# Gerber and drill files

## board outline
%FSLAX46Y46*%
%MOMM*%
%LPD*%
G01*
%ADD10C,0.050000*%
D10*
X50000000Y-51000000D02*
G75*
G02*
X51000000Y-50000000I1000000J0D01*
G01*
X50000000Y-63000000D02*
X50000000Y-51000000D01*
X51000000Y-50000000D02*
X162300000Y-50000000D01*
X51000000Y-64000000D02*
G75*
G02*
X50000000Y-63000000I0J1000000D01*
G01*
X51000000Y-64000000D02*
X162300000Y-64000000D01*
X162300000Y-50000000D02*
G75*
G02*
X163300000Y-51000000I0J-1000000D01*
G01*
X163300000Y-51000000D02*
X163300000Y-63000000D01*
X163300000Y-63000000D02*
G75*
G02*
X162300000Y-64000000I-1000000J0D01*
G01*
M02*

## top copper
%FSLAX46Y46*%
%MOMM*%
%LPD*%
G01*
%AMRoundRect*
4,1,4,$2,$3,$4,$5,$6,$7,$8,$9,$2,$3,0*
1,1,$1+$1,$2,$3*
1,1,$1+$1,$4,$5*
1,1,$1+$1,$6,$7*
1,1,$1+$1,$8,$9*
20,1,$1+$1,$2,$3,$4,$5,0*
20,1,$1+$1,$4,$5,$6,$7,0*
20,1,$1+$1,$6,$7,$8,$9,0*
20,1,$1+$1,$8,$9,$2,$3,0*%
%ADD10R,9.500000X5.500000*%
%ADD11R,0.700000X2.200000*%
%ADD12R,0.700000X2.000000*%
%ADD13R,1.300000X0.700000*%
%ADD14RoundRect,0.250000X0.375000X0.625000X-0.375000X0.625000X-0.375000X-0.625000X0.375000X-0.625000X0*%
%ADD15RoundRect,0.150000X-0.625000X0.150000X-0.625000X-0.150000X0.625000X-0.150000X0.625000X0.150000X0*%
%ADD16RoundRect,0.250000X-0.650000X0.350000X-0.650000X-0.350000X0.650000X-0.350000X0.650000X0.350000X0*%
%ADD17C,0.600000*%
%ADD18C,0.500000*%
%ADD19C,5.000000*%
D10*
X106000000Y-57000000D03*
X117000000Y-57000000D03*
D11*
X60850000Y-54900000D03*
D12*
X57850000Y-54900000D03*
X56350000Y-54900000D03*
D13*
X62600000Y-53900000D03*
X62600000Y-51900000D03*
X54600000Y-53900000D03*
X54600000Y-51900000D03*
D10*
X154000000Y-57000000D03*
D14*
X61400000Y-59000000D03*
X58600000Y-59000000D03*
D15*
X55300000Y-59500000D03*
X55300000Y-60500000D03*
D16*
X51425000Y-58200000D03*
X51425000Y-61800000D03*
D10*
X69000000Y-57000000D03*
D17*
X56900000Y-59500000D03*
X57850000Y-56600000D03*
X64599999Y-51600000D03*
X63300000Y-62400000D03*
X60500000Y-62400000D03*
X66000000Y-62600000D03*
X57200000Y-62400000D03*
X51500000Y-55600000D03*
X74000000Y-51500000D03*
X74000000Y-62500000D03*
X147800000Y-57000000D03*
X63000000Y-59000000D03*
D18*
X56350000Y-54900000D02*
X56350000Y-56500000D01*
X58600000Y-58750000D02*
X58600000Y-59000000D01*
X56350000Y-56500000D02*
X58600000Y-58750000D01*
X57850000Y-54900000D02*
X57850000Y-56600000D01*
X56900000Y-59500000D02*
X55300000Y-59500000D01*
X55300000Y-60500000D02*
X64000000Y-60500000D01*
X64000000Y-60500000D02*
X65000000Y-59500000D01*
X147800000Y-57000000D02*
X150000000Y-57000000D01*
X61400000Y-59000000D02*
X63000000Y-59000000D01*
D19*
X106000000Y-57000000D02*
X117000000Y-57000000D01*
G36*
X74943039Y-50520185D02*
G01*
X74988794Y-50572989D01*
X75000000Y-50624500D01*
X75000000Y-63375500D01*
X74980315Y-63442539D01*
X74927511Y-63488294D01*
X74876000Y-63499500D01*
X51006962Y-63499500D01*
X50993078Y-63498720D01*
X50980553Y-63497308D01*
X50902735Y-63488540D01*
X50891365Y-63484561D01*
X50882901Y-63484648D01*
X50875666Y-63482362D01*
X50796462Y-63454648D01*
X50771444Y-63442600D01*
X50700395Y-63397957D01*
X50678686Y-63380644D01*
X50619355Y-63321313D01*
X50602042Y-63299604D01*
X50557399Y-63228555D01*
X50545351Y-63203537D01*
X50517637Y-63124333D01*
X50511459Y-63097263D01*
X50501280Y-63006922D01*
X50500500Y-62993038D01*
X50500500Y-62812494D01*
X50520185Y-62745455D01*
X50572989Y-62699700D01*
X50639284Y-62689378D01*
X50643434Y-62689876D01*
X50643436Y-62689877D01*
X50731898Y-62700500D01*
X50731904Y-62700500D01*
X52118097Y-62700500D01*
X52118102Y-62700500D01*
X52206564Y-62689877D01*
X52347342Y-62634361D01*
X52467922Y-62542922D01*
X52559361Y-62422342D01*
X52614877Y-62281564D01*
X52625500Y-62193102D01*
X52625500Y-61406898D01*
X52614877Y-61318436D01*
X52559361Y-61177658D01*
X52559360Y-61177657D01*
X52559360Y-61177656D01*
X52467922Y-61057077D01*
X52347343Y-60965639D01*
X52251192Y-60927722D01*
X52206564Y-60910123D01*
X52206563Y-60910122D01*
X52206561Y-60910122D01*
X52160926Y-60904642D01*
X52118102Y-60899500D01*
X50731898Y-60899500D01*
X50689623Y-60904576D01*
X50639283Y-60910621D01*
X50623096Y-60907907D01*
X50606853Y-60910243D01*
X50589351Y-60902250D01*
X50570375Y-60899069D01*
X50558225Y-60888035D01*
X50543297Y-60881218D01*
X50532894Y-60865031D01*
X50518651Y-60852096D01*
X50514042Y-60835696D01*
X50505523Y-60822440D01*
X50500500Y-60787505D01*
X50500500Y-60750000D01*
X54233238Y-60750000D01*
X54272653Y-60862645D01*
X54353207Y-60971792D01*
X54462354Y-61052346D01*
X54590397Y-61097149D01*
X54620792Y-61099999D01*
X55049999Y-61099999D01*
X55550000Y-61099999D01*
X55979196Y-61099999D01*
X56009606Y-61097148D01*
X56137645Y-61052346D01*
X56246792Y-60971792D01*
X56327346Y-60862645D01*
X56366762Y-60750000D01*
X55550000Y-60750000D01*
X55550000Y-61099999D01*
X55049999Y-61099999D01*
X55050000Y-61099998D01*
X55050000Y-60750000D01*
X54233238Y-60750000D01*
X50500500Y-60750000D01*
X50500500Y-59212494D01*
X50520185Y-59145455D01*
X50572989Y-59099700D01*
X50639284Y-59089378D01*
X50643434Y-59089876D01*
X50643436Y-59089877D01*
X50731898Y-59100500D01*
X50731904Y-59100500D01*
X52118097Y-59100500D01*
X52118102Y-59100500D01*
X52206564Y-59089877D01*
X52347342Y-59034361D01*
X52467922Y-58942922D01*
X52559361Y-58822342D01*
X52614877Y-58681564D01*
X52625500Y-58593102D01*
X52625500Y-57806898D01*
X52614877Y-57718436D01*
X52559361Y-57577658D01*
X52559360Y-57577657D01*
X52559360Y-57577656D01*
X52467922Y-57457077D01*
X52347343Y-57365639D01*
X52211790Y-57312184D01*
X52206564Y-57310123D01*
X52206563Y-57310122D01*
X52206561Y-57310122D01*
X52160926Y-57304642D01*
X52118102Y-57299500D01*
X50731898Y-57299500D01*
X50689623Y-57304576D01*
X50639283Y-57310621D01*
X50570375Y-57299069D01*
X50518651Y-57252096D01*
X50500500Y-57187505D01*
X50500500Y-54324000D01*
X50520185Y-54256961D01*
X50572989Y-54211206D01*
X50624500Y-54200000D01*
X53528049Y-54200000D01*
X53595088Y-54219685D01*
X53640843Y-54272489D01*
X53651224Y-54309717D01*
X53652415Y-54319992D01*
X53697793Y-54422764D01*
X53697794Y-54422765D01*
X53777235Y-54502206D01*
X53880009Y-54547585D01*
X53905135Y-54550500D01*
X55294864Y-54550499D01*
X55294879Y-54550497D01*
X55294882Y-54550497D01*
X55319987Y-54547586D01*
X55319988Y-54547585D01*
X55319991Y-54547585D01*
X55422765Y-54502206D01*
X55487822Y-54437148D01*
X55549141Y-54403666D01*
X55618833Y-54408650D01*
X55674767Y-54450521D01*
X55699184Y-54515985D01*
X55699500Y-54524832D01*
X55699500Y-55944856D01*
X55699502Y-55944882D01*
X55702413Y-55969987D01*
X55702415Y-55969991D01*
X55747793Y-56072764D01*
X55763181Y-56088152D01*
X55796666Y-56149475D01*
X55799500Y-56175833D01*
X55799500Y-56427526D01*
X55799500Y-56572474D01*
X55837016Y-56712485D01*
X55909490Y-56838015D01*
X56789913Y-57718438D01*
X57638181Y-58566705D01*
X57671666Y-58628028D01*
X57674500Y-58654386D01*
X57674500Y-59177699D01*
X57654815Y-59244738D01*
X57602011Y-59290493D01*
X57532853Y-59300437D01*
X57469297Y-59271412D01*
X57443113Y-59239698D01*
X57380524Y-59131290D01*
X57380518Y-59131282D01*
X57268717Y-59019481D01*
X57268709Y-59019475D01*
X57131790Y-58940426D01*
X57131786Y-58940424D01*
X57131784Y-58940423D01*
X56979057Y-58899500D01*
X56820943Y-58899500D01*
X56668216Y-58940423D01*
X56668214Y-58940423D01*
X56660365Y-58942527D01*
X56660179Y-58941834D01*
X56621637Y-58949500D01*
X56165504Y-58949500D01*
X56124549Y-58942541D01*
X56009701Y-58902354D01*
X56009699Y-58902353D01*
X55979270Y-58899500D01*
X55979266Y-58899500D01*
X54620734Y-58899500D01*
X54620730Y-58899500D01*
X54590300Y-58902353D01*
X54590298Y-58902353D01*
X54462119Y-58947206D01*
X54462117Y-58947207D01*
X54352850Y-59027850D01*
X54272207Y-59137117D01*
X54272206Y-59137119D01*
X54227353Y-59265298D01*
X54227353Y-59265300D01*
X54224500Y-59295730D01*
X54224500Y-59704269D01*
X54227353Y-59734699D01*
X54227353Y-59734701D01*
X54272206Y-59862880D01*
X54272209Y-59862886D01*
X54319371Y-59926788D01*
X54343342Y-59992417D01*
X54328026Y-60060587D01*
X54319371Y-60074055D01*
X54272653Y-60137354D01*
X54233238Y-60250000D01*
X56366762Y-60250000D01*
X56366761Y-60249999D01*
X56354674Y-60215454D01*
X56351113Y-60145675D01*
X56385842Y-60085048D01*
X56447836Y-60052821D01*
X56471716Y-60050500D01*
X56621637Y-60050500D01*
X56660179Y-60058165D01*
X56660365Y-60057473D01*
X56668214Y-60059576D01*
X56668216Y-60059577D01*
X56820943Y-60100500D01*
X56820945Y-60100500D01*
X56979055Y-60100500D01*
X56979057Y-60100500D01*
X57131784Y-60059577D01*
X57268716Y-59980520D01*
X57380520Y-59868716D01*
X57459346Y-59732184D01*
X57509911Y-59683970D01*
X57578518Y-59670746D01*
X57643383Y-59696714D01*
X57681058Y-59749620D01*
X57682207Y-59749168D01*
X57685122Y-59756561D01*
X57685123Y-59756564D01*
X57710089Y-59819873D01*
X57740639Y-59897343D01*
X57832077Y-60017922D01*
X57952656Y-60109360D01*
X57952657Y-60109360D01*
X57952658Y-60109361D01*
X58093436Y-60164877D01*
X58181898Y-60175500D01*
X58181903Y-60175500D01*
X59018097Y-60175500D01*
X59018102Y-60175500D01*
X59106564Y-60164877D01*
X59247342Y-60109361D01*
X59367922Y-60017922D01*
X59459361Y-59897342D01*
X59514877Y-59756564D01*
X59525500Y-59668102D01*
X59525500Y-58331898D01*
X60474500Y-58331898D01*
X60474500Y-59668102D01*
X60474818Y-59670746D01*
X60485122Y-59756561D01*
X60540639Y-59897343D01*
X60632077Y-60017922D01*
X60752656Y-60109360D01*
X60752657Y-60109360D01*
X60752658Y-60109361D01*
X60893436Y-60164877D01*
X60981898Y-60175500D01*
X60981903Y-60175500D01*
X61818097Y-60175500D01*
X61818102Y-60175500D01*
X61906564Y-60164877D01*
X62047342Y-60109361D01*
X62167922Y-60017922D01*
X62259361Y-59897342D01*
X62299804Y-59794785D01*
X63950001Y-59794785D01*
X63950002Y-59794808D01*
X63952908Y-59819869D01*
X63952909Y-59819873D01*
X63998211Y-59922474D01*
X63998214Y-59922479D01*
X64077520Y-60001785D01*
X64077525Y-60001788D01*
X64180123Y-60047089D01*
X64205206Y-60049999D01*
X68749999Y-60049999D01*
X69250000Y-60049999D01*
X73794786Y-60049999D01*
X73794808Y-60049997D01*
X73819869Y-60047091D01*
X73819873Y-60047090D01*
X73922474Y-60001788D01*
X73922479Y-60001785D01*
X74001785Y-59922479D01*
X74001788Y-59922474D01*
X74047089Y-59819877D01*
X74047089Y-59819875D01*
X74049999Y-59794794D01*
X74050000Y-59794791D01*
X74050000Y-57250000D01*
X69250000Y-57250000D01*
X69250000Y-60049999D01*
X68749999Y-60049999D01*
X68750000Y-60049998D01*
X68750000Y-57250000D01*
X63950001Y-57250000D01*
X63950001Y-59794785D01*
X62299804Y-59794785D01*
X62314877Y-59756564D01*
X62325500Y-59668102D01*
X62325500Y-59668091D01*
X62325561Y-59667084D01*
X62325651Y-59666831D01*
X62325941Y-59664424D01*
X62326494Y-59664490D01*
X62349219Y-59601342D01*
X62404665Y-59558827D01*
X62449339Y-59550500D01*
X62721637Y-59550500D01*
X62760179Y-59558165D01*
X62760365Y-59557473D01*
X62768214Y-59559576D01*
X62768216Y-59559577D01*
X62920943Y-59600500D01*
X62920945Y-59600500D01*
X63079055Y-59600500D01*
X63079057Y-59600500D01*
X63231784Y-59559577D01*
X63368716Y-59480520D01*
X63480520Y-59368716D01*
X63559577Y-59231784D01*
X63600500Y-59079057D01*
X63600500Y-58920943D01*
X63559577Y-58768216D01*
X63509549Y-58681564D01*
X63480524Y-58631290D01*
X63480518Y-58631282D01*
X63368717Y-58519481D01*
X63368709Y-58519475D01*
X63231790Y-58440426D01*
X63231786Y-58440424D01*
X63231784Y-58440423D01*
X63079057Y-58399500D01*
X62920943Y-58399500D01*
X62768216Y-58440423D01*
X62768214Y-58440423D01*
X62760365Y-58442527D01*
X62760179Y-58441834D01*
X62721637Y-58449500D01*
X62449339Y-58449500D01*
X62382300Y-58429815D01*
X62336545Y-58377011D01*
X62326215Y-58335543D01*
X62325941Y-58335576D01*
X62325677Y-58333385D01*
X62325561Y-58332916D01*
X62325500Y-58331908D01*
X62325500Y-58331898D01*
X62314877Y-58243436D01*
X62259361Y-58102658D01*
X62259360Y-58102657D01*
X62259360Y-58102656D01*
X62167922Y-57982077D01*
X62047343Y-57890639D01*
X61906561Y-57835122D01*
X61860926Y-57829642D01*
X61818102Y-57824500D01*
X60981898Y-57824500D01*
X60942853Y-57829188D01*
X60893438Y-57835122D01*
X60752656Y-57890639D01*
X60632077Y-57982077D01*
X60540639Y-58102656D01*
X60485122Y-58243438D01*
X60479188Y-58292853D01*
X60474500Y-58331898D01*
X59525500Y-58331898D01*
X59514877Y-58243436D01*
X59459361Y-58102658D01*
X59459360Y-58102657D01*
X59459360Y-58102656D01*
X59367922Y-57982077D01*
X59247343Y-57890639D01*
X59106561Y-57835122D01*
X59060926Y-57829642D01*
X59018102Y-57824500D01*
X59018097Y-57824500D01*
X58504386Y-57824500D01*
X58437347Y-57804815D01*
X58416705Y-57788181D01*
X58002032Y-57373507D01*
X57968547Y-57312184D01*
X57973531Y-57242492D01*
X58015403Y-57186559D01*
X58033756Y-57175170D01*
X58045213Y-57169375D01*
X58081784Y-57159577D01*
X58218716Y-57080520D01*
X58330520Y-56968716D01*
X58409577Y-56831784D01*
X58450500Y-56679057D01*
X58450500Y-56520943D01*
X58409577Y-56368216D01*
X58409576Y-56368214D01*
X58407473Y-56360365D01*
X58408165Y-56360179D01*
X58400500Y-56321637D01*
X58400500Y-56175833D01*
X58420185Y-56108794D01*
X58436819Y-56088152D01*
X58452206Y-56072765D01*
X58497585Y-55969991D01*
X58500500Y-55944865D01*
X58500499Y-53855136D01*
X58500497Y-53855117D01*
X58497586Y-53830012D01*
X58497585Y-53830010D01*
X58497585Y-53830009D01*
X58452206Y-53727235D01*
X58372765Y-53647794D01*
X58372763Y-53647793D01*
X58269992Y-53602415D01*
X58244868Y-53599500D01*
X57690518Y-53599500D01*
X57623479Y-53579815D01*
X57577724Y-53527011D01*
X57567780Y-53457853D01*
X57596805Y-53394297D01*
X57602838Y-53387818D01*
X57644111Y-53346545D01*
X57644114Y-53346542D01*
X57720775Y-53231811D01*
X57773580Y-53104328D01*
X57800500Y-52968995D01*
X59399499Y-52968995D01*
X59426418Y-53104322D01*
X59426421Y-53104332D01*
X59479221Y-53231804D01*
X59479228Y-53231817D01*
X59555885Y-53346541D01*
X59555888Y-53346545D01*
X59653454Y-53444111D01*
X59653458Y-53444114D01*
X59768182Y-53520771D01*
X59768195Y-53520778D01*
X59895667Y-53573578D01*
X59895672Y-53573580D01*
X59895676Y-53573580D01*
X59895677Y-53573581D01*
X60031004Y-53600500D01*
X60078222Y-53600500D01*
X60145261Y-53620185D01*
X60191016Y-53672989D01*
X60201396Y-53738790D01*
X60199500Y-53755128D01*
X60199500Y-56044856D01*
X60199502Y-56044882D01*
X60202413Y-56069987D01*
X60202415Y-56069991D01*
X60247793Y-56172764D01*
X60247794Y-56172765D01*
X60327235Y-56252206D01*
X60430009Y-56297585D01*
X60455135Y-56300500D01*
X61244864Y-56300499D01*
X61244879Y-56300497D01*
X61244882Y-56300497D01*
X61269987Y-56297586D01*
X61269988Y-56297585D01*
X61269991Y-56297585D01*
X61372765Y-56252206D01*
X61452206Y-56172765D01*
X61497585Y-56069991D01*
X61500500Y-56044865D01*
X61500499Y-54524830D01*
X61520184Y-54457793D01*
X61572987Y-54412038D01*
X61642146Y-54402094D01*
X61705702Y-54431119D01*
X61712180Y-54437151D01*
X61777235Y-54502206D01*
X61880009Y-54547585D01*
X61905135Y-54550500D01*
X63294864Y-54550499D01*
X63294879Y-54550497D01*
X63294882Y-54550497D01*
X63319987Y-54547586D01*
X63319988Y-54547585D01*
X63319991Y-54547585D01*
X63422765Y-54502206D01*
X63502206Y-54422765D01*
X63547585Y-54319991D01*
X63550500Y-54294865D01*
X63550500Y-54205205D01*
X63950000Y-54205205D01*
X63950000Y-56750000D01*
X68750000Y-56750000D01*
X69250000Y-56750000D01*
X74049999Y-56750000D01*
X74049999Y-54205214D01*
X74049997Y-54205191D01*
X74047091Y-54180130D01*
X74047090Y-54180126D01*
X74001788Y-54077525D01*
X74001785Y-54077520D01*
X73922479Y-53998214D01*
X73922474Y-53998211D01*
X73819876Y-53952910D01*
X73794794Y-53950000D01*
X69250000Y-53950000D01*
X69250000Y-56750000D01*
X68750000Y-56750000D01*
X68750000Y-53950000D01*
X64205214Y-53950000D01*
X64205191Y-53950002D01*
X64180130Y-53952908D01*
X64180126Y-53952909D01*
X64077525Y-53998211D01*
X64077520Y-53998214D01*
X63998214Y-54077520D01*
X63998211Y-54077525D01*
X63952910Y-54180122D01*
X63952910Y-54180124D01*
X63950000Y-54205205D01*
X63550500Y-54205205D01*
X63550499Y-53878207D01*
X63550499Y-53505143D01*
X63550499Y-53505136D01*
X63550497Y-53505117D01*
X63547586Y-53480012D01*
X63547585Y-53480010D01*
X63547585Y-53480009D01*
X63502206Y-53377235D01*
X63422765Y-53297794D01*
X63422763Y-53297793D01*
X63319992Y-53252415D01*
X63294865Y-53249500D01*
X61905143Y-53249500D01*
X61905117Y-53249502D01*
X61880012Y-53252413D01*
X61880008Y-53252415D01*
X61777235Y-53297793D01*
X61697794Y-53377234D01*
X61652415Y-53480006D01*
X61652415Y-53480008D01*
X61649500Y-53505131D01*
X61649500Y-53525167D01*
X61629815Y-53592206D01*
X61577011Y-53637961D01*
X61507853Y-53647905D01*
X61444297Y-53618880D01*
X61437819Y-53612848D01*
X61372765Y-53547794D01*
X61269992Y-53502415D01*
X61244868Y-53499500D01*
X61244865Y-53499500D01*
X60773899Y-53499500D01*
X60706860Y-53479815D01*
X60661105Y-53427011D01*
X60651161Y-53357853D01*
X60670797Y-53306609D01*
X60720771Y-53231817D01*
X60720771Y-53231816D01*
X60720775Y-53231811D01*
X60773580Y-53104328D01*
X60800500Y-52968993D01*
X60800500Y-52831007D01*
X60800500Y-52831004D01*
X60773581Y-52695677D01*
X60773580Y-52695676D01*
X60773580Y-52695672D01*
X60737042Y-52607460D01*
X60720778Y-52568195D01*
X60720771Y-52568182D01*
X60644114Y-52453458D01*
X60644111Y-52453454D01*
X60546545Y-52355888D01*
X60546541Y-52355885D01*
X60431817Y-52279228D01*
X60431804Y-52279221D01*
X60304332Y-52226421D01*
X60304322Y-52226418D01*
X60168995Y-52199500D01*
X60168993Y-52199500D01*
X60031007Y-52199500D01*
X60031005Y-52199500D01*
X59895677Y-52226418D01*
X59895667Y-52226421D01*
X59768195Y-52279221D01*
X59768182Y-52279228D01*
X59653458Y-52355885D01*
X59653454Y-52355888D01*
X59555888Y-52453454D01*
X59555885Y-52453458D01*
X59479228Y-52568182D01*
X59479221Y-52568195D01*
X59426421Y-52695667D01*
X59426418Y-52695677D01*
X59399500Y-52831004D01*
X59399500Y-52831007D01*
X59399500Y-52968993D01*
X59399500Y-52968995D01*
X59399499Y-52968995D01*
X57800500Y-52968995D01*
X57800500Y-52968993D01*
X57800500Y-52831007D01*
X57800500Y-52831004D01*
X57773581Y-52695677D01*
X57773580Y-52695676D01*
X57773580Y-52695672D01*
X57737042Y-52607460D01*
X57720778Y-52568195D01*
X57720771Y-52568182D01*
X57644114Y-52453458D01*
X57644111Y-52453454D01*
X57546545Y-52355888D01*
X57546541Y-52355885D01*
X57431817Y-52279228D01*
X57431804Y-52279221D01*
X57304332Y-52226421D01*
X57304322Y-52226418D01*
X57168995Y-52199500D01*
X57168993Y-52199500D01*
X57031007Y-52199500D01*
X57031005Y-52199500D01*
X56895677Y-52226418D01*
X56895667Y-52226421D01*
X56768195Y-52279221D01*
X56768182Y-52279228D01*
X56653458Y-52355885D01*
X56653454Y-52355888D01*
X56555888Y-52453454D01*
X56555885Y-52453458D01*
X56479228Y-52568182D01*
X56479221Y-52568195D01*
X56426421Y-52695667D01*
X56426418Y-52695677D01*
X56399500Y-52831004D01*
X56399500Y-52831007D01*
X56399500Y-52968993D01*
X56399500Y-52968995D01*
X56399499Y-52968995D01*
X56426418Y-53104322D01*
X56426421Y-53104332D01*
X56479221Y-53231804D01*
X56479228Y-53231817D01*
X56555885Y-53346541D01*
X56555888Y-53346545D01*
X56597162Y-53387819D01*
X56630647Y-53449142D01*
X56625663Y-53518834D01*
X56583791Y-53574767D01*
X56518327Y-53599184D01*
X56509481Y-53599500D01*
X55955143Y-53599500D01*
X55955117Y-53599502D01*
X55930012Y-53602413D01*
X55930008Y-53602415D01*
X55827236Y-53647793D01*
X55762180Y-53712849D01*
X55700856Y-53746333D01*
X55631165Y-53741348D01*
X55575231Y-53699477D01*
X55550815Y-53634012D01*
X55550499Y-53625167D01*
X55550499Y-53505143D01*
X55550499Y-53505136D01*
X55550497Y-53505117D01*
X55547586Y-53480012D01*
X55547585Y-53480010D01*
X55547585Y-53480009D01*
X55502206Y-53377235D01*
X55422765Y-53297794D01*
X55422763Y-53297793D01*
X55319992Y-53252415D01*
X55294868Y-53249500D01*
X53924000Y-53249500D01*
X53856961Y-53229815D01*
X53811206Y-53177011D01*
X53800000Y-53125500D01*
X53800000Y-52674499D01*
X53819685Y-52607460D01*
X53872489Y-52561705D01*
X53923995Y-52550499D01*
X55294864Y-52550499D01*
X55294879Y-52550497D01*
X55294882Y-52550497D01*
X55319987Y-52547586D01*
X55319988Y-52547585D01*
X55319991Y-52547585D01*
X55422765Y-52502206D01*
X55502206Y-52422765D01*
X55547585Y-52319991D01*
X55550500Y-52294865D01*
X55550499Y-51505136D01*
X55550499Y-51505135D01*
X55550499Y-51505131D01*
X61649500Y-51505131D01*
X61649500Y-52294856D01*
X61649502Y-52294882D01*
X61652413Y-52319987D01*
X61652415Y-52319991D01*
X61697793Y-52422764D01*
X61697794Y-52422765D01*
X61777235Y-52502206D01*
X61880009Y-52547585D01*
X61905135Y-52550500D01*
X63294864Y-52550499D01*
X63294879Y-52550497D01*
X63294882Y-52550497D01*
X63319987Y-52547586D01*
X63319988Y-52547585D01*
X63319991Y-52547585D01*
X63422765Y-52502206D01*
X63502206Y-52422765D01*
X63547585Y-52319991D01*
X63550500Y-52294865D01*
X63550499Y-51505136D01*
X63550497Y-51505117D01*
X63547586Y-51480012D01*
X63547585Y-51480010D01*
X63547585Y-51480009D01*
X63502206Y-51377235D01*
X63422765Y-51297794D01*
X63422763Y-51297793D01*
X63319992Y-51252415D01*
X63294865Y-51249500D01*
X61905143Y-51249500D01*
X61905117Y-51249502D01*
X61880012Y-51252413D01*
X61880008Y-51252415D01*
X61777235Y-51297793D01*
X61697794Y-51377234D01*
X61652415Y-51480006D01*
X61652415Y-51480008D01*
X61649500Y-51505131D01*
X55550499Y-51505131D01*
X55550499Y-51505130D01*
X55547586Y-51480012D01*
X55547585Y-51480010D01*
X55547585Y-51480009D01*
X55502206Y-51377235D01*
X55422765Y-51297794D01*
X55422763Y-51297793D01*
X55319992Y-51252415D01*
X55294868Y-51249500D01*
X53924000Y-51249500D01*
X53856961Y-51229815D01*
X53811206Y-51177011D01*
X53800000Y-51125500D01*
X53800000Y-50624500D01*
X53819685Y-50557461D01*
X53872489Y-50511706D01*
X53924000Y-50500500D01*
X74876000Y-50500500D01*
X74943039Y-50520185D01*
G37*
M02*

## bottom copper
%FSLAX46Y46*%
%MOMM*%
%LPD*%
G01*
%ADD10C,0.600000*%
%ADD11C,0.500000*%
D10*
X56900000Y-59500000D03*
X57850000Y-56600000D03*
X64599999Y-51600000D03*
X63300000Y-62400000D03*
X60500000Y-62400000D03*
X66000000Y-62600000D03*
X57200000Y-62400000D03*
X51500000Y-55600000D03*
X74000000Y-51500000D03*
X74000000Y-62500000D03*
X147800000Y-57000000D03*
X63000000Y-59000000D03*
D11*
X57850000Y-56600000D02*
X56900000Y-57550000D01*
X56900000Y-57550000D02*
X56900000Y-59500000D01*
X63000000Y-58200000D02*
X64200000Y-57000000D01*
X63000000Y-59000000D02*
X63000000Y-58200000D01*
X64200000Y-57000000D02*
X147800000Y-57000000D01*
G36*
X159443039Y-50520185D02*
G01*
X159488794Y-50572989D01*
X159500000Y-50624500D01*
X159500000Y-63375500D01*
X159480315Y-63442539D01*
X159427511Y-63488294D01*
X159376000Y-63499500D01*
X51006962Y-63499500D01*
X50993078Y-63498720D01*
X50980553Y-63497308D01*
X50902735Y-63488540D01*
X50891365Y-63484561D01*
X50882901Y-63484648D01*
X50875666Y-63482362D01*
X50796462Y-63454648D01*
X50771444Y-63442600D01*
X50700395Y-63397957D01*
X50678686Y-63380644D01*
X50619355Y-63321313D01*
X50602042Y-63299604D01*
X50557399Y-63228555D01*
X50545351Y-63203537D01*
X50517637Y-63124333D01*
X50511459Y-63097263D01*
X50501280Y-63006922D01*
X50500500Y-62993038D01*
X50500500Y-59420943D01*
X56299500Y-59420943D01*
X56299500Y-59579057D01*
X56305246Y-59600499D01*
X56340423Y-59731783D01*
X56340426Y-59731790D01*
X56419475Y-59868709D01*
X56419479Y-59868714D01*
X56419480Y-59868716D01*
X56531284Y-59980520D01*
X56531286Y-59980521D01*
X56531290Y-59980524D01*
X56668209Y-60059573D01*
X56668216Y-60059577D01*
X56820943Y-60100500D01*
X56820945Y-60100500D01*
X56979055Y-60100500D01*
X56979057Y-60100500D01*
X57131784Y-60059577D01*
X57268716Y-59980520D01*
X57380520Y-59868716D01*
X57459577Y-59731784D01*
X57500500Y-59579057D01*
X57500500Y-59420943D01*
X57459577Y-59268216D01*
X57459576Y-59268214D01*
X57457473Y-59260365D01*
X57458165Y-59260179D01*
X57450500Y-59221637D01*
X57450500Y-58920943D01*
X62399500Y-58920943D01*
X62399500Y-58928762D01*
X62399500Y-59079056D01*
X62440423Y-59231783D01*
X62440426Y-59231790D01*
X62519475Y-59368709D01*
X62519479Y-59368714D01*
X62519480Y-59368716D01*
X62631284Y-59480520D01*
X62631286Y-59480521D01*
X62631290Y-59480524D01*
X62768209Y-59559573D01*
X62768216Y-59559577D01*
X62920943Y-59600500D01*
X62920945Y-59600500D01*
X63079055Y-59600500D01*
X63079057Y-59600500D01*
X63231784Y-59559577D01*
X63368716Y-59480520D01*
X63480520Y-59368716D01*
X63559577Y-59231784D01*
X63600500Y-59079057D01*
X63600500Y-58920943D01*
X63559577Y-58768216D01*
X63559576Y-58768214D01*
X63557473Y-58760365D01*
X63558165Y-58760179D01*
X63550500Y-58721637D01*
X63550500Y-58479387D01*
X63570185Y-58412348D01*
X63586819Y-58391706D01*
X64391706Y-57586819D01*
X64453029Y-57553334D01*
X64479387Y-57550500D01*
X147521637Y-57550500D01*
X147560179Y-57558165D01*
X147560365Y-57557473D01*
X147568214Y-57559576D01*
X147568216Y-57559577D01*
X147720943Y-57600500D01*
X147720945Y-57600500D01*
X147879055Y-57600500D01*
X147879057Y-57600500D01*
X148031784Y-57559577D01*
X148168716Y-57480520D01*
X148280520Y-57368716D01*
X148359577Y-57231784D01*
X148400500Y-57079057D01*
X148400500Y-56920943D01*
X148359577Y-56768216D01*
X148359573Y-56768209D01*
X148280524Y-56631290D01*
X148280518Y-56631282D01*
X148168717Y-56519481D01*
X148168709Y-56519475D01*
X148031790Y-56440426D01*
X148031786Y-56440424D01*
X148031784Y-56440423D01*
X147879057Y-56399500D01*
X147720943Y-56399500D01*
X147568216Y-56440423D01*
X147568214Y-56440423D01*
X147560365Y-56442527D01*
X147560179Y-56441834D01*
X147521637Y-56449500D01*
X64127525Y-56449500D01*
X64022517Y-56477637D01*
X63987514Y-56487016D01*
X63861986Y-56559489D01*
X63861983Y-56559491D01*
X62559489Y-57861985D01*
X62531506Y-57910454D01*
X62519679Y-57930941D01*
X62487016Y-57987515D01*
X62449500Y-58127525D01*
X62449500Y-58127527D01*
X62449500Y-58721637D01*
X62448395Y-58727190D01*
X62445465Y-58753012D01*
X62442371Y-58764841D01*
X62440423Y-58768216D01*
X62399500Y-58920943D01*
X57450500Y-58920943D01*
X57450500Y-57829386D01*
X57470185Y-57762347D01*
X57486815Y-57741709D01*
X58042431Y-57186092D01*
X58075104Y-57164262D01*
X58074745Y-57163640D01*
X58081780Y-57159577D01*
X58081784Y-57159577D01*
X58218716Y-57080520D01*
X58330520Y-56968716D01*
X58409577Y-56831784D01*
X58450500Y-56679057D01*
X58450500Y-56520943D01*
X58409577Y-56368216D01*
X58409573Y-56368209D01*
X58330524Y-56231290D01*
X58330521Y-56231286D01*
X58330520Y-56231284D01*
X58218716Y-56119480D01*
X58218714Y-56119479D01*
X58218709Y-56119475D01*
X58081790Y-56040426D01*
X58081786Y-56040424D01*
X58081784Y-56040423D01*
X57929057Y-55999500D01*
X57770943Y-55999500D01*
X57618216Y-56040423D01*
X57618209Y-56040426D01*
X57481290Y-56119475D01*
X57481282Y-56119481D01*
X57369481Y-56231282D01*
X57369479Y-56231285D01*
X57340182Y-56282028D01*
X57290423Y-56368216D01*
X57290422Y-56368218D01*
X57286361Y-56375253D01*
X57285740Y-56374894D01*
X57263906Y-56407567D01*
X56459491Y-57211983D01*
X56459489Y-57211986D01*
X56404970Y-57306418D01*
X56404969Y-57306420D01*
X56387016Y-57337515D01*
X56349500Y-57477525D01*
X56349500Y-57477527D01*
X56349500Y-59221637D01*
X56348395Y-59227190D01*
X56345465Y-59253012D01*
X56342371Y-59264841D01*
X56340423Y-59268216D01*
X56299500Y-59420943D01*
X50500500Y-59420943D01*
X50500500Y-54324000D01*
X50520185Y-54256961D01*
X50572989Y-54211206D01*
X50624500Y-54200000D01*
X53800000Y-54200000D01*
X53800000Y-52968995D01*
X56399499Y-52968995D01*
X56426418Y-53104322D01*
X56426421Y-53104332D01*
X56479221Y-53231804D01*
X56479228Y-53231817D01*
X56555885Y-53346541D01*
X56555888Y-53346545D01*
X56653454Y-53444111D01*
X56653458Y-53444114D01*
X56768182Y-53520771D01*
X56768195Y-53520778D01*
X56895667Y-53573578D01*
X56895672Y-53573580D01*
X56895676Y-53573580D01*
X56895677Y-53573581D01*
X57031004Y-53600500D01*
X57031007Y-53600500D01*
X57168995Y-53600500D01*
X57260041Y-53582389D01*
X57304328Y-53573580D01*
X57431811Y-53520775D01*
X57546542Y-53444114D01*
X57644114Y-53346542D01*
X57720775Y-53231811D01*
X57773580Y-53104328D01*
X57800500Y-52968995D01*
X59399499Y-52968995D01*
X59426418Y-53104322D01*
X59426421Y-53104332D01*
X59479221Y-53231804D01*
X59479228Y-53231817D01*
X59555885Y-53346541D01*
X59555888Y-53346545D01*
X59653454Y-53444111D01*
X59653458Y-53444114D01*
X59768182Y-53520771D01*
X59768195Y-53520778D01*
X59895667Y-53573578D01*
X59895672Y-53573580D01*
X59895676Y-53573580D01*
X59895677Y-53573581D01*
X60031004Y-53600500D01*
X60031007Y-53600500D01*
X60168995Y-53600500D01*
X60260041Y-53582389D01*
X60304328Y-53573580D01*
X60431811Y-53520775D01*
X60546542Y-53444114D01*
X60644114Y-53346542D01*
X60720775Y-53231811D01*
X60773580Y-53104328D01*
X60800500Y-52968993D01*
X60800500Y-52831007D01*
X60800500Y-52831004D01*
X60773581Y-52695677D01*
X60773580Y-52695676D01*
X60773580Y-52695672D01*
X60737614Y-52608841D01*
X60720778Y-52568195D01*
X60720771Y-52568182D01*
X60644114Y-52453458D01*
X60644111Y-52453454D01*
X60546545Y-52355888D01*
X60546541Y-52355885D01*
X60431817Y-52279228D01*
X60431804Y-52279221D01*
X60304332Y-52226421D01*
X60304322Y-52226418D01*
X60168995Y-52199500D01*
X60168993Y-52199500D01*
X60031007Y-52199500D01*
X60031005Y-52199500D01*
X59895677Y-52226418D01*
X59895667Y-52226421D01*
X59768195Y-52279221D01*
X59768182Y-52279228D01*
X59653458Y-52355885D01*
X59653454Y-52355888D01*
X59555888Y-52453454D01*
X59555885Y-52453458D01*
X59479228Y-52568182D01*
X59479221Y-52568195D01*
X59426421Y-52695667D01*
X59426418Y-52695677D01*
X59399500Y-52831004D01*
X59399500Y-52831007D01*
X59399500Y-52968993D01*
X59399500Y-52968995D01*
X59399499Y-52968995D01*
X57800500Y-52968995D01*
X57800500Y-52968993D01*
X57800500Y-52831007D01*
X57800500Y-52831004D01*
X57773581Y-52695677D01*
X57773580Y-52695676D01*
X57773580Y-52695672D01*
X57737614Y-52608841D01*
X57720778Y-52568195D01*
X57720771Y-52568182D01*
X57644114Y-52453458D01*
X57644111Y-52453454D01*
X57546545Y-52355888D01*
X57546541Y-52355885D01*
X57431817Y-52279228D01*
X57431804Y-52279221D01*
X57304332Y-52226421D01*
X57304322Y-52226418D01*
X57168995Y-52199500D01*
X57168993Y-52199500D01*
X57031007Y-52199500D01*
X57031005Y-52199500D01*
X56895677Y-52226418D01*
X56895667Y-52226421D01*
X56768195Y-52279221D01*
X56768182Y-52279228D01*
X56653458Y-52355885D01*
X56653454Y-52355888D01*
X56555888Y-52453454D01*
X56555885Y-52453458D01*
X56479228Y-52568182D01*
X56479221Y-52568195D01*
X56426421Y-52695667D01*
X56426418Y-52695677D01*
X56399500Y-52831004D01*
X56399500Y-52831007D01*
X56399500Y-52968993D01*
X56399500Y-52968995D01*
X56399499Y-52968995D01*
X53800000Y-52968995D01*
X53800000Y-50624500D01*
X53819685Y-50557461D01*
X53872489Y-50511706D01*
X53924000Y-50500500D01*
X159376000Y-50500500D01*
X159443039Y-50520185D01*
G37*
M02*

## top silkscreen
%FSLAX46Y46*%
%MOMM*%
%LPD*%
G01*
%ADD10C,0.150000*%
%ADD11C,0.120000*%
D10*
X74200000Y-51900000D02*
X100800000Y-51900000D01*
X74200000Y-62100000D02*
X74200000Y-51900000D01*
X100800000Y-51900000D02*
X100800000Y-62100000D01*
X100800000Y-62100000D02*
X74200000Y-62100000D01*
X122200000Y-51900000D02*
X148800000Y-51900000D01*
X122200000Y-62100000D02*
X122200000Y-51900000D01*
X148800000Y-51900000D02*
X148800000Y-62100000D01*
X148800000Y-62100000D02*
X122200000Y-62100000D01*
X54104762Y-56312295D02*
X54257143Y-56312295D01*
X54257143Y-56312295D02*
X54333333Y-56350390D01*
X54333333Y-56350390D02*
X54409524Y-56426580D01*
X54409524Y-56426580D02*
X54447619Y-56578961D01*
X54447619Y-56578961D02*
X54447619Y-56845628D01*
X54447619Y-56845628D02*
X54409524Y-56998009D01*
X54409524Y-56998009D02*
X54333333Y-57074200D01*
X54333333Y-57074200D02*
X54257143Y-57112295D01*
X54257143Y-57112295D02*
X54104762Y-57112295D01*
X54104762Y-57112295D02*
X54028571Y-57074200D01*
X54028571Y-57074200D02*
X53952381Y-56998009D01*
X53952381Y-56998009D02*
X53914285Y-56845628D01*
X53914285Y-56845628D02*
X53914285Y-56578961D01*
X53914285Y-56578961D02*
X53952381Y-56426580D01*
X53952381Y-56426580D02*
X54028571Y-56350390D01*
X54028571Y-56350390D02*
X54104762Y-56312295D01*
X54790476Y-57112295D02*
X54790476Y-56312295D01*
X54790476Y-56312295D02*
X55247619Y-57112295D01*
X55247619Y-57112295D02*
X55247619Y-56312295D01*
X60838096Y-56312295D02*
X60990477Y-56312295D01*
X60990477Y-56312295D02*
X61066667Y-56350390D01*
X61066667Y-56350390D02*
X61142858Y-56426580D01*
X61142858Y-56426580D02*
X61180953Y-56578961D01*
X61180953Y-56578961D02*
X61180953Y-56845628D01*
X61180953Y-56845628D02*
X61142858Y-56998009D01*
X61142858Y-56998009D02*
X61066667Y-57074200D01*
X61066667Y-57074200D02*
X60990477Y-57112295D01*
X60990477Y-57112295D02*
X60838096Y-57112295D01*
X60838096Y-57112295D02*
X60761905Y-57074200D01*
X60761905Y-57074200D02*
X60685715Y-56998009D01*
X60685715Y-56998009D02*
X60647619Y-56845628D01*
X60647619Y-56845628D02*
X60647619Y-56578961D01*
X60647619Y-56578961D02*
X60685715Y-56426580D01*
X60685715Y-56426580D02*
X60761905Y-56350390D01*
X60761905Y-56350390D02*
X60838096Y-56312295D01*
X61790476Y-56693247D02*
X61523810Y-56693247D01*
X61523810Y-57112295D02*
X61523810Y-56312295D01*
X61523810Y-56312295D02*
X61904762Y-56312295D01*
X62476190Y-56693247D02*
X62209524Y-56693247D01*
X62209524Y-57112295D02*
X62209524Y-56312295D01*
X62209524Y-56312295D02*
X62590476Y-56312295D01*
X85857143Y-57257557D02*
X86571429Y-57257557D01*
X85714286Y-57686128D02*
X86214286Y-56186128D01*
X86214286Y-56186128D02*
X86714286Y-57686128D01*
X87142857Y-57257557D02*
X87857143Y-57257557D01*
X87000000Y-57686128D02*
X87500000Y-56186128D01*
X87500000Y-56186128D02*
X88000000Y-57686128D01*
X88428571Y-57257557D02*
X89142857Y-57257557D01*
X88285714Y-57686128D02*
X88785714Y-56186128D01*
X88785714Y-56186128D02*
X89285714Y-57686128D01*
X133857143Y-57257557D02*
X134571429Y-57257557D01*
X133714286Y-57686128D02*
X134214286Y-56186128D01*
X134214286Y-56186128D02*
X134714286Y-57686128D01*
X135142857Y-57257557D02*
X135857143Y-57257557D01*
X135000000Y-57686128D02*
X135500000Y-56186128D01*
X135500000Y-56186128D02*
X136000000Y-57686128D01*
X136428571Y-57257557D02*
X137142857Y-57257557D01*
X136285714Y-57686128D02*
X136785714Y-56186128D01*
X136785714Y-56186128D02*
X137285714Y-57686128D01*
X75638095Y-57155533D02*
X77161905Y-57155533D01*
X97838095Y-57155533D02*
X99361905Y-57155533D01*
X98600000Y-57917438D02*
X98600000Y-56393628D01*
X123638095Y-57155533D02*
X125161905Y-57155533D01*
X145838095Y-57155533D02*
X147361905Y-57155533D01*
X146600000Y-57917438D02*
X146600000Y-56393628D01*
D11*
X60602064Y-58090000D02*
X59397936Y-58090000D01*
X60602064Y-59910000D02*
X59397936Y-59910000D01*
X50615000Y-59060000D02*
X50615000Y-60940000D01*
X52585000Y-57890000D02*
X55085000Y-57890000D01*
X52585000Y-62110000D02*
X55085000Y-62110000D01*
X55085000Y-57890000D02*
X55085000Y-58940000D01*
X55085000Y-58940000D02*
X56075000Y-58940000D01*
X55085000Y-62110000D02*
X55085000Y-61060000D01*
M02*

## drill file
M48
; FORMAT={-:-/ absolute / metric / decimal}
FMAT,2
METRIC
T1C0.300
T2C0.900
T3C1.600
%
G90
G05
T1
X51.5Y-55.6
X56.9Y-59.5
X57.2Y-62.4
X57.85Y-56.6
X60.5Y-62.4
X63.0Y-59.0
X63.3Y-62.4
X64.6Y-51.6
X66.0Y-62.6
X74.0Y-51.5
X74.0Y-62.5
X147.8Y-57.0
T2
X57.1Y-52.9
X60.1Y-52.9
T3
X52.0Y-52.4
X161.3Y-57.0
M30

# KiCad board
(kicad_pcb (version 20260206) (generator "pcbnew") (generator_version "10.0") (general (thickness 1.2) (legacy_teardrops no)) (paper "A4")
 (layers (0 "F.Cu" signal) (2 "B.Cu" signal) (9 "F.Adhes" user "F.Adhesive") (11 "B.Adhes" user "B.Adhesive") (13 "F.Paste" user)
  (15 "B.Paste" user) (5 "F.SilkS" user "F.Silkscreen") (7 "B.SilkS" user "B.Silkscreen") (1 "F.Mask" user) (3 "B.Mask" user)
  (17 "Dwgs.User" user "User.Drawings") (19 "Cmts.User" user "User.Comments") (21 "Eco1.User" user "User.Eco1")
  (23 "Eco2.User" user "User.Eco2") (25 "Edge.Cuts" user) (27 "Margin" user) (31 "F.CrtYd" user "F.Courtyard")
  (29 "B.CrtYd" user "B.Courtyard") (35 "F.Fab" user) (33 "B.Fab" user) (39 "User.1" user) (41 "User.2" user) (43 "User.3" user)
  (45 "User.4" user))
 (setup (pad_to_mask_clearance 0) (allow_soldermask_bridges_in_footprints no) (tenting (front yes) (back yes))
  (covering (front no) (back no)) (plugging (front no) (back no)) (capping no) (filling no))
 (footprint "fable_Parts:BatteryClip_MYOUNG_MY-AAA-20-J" (layer "F.Cu") (at 106 57 180)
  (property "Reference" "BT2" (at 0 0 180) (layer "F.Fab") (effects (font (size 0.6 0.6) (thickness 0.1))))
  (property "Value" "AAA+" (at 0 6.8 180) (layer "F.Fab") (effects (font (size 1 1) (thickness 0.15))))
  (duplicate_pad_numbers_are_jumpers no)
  (pad "1" smd rect (at 0 0 180) (size 9.5 5.5) (layers "F.Cu" "F.Mask" "F.Paste") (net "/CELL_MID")))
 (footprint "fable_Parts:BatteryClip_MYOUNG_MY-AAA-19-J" (layer "F.Cu") (at 117 57)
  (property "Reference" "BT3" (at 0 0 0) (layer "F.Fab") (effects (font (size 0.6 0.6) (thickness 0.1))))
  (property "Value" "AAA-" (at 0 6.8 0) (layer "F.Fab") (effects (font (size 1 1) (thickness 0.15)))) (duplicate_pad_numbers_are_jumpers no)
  (pad "1" smd rect (at 0 0) (size 9.5 5.5) (layers "F.Cu" "F.Mask" "F.Paste") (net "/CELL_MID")))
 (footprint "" (layer "F.Cu") (at 52 52.4)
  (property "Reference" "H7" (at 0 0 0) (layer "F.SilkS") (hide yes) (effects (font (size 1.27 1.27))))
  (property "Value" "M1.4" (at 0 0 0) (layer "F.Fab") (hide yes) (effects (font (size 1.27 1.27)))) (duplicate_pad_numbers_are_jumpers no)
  (pad "" np_thru_hole circle (at 0 0) (size 1.6 1.6) (drill 1.6) (layers "*.Cu")))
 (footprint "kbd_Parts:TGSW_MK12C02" (layer "F.Cu") (at 58.6 52.9 180)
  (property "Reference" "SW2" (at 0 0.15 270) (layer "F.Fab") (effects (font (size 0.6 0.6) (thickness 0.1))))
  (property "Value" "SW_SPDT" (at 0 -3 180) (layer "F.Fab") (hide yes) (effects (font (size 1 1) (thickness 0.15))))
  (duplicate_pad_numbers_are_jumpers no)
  (pad "" np_thru_hole circle (at -1.5 0 180) (size 0.9 0.9) (drill 0.9) (layers "*.Cu" "*.Mask"))
  (pad "" np_thru_hole circle (at 1.5 0 180) (size 0.9 0.9) (drill 0.9) (layers "*.Cu" "*.Mask"))
  (pad "1" smd rect (at -2.25 -2 180) (size 0.7 2.2) (layers "F.Cu" "F.Mask" "F.Paste") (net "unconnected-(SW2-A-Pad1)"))
  (pad "2" smd rect (at 0.75 -2 180) (size 0.7 2) (layers "F.Cu" "F.Mask" "F.Paste") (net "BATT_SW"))
  (pad "3" smd rect (at 2.25 -2 180) (size 0.7 2) (layers "F.Cu" "F.Mask" "F.Paste") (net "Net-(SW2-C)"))
  (pad "4" smd rect (at -4 -1 90) (size 0.7 1.3) (layers "F.Cu" "F.Mask" "F.Paste"))
  (pad "4" smd rect (at -4 1 90) (size 0.7 1.3) (layers "F.Cu" "F.Mask" "F.Paste"))
  (pad "4" smd rect (at 4 -1 90) (size 0.7 1.3) (layers "F.Cu" "F.Mask" "F.Paste"))
  (pad "4" smd rect (at 4 1 90) (size 0.7 1.3) (layers "F.Cu" "F.Mask" "F.Paste")))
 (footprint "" (layer "F.Cu") (at 161.3 57)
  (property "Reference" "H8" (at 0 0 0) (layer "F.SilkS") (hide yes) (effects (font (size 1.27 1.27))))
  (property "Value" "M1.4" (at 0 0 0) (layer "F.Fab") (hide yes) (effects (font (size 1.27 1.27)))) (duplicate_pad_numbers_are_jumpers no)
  (pad "" np_thru_hole circle (at 0 0) (size 1.6 1.6) (drill 1.6) (layers "*.Cu")))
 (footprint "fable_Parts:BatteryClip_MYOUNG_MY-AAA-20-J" (layer "F.Cu") (at 154 57 180)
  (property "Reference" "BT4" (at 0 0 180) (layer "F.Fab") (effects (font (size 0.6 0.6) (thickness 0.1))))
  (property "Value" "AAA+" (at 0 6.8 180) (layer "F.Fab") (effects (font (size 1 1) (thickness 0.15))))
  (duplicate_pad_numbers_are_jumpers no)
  (pad "1" smd rect (at 0 0 180) (size 9.5 5.5) (layers "F.Cu" "F.Mask" "F.Paste") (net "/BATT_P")))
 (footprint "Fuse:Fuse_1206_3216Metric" (layer "F.Cu") (at 60 59 180)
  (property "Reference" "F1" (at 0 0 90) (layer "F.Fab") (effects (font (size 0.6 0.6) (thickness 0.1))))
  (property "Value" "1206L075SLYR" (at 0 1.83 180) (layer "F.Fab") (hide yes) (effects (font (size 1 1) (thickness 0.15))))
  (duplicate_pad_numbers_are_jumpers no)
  (fp_line (start -0.602064 0.91) (end 0.602064 0.91) (stroke (width 0.12) (type solid)) (layer "F.SilkS"))
  (fp_line (start -0.602064 -0.91) (end 0.602064 -0.91) (stroke (width 0.12) (type solid)) (layer "F.SilkS"))
  (pad "1" smd roundrect (at -1.4 0 180) (size 1.25 1.75) (layers "F.Cu" "F.Mask" "F.Paste") (roundrect_rratio 0.2) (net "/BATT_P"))
  (pad "2" smd roundrect (at 1.4 0 180) (size 1.25 1.75) (layers "F.Cu" "F.Mask" "F.Paste") (roundrect_rratio 0.2) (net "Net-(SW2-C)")))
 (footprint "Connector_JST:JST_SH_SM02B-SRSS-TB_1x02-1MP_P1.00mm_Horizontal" (layer "F.Cu") (at 53.3 60 -90)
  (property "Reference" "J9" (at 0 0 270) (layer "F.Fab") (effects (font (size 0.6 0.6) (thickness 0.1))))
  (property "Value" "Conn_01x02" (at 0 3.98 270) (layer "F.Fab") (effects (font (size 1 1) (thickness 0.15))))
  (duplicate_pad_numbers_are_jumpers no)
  (fp_line (start -0.94 2.685) (end 0.94 2.685) (stroke (width 0.12) (type solid)) (layer "F.SilkS"))
  (fp_line (start -2.11 0.715) (end -2.11 -1.785) (stroke (width 0.12) (type solid)) (layer "F.SilkS"))
  (fp_line (start 2.11 0.715) (end 2.11 -1.785) (stroke (width 0.12) (type solid)) (layer "F.SilkS"))
  (fp_line (start -2.11 -1.785) (end -1.06 -1.785) (stroke (width 0.12) (type solid)) (layer "F.SilkS"))
  (fp_line (start -1.06 -1.785) (end -1.06 -2.775) (stroke (width 0.12) (type solid)) (layer "F.SilkS"))
  (fp_line (start 2.11 -1.785) (end 1.06 -1.785) (stroke (width 0.12) (type solid)) (layer "F.SilkS"))
  (pad "1" smd roundrect (at -0.5 -2 270) (size 0.6 1.55) (layers "F.Cu" "F.Mask" "F.Paste") (roundrect_rratio 0.25) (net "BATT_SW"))
  (pad "2" smd roundrect (at 0.5 -2 270) (size 0.6 1.55) (layers "F.Cu" "F.Mask" "F.Paste") (roundrect_rratio 0.25) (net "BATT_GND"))
  (pad "MP" smd roundrect (at -1.8 1.875 270) (size 1.2 1.8) (layers "F.Cu" "F.Mask" "F.Paste") (roundrect_rratio 0.208333))
  (pad "MP" smd roundrect (at 1.8 1.875 270) (size 1.2 1.8) (layers "F.Cu" "F.Mask" "F.Paste") (roundrect_rratio 0.208333)))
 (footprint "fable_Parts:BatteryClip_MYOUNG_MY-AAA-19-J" (layer "F.Cu") (at 69 57)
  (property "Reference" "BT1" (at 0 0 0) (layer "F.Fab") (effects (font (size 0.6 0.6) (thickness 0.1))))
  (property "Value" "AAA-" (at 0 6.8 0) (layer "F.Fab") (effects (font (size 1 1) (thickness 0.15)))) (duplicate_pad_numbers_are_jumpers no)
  (pad "1" smd rect (at 0 0) (size 9.5 5.5) (layers "F.Cu" "F.Mask" "F.Paste") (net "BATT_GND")))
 (gr_line (start 74.2 51.9) (end 100.8 51.9) (stroke (width 0.15) (type default)) (layer "F.SilkS"))
 (gr_line (start 74.2 62.1) (end 74.2 51.9) (stroke (width 0.15) (type default)) (layer "F.SilkS"))
 (gr_line (start 100.8 51.9) (end 100.8 62.1) (stroke (width 0.15) (type default)) (layer "F.SilkS"))
 (gr_line (start 100.8 62.1) (end 74.2 62.1) (stroke (width 0.15) (type default)) (layer "F.SilkS"))
 (gr_line (start 122.2 51.9) (end 148.8 51.9) (stroke (width 0.15) (type default)) (layer "F.SilkS"))
 (gr_line (start 122.2 62.1) (end 122.2 51.9) (stroke (width 0.15) (type default)) (layer "F.SilkS"))
 (gr_line (start 148.8 51.9) (end 148.8 62.1) (stroke (width 0.15) (type default)) (layer "F.SilkS"))
 (gr_line (start 148.8 62.1) (end 122.2 62.1) (stroke (width 0.15) (type default)) (layer "F.SilkS"))
 (gr_arc (start 50 51) (mid 50.292893 50.292893) (end 51 50) (stroke (width 0.05) (type default)) (layer "Edge.Cuts"))
 (gr_line (start 50 63) (end 50 51) (stroke (width 0.05) (type default)) (layer "Edge.Cuts"))
 (gr_line (start 51 50) (end 162.3 50) (stroke (width 0.05) (type default)) (layer "Edge.Cuts"))
 (gr_arc (start 51 64) (mid 50.292893 63.707106) (end 50 63) (stroke (width 0.05) (type default)) (layer "Edge.Cuts"))
 (gr_line (start 51 64) (end 162.3 64) (stroke (width 0.05) (type default)) (layer "Edge.Cuts"))
 (gr_arc (start 162.3 50) (mid 163.007106 50.292893) (end 163.3 51) (stroke (width 0.05) (type default)) (layer "Edge.Cuts"))
 (gr_line (start 163.3 51) (end 163.3 63) (stroke (width 0.05) (type default)) (layer "Edge.Cuts"))
 (gr_arc (start 163.3 63) (mid 163.007106 63.707106) (end 162.3 64) (stroke (width 0.05) (type default)) (layer "Edge.Cuts"))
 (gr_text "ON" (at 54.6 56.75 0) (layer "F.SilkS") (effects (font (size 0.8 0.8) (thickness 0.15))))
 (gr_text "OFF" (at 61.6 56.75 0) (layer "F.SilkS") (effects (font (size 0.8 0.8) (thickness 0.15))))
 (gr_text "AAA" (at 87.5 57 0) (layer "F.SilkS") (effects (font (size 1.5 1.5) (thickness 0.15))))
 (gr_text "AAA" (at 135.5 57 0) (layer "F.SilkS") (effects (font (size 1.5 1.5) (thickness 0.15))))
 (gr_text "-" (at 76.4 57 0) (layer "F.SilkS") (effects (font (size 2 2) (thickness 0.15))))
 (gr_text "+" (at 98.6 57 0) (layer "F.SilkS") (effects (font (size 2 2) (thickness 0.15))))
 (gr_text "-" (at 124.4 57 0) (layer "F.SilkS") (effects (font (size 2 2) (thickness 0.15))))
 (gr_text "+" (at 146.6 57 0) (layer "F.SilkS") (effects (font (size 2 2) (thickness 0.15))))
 (segment (start 56.35 54.9) (end 56.35 56.5) (width 0.5) (layer "F.Cu") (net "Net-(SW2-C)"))
 (segment (start 58.6 58.75) (end 58.6 59) (width 0.5) (layer "F.Cu") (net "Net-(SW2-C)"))
 (segment (start 56.35 56.5) (end 58.6 58.75) (width 0.5) (layer "F.Cu") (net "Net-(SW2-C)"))
 (segment (start 57.85 54.9) (end 57.85 56.6) (width 0.5) (layer "F.Cu") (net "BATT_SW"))
 (segment (start 56.9 59.5) (end 55.3 59.5) (width 0.5) (layer "F.Cu") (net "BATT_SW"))
 (via (at 56.9 59.5) (size 0.6) (drill 0.3) (layers "F.Cu" "B.Cu") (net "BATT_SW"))
 (via (at 57.85 56.6) (size 0.6) (drill 0.3) (layers "F.Cu" "B.Cu") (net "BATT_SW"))
 (segment (start 57.85 56.6) (end 56.9 57.55) (width 0.5) (layer "B.Cu") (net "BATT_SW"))
 (segment (start 56.9 57.55) (end 56.9 59.5) (width 0.5) (layer "B.Cu") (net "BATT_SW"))
 (segment (start 55.3 60.5) (end 64 60.5) (width 0.5) (layer "F.Cu") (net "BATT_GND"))
 (segment (start 64 60.5) (end 65 59.5) (width 0.5) (layer "F.Cu") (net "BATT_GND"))
 (via (at 64.599999 51.6) (size 0.6) (drill 0.3) (layers "F.Cu" "B.Cu") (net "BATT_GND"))
 (via (at 63.3 62.4) (size 0.6) (drill 0.3) (layers "F.Cu" "B.Cu") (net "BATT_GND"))
 (via (at 60.5 62.4) (size 0.6) (drill 0.3) (layers "F.Cu" "B.Cu") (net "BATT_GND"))
 (via (at 66 62.6) (size 0.6) (drill 0.3) (layers "F.Cu" "B.Cu") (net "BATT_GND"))
 (via (at 57.2 62.4) (size 0.6) (drill 0.3) (layers "F.Cu" "B.Cu") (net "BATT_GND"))
 (via (at 51.5 55.6) (size 0.6) (drill 0.3) (layers "F.Cu" "B.Cu") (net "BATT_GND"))
 (via (at 74 51.5) (size 0.6) (drill 0.3) (layers "F.Cu" "B.Cu") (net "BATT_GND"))
 (via (at 74 62.5) (size 0.6) (drill 0.3) (layers "F.Cu" "B.Cu") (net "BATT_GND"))
 (segment (start 147.8 57) (end 150 57) (width 0.5) (layer "F.Cu") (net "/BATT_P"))
 (segment (start 61.4 59) (end 63 59) (width 0.5) (layer "F.Cu") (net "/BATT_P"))
 (via (at 147.8 57) (size 0.6) (drill 0.3) (layers "F.Cu" "B.Cu") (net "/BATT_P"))
 (via (at 63 59) (size 0.6) (drill 0.3) (layers "F.Cu" "B.Cu") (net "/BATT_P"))
 (segment (start 63 58.2) (end 64.2 57) (width 0.5) (layer "B.Cu") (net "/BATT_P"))
 (segment (start 63 59) (end 63 58.2) (width 0.5) (layer "B.Cu") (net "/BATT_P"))
 (segment (start 64.2 57) (end 147.8 57) (width 0.5) (layer "B.Cu") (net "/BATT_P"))
 (segment (start 106 57) (end 117 57) (width 5) (layer "F.Cu") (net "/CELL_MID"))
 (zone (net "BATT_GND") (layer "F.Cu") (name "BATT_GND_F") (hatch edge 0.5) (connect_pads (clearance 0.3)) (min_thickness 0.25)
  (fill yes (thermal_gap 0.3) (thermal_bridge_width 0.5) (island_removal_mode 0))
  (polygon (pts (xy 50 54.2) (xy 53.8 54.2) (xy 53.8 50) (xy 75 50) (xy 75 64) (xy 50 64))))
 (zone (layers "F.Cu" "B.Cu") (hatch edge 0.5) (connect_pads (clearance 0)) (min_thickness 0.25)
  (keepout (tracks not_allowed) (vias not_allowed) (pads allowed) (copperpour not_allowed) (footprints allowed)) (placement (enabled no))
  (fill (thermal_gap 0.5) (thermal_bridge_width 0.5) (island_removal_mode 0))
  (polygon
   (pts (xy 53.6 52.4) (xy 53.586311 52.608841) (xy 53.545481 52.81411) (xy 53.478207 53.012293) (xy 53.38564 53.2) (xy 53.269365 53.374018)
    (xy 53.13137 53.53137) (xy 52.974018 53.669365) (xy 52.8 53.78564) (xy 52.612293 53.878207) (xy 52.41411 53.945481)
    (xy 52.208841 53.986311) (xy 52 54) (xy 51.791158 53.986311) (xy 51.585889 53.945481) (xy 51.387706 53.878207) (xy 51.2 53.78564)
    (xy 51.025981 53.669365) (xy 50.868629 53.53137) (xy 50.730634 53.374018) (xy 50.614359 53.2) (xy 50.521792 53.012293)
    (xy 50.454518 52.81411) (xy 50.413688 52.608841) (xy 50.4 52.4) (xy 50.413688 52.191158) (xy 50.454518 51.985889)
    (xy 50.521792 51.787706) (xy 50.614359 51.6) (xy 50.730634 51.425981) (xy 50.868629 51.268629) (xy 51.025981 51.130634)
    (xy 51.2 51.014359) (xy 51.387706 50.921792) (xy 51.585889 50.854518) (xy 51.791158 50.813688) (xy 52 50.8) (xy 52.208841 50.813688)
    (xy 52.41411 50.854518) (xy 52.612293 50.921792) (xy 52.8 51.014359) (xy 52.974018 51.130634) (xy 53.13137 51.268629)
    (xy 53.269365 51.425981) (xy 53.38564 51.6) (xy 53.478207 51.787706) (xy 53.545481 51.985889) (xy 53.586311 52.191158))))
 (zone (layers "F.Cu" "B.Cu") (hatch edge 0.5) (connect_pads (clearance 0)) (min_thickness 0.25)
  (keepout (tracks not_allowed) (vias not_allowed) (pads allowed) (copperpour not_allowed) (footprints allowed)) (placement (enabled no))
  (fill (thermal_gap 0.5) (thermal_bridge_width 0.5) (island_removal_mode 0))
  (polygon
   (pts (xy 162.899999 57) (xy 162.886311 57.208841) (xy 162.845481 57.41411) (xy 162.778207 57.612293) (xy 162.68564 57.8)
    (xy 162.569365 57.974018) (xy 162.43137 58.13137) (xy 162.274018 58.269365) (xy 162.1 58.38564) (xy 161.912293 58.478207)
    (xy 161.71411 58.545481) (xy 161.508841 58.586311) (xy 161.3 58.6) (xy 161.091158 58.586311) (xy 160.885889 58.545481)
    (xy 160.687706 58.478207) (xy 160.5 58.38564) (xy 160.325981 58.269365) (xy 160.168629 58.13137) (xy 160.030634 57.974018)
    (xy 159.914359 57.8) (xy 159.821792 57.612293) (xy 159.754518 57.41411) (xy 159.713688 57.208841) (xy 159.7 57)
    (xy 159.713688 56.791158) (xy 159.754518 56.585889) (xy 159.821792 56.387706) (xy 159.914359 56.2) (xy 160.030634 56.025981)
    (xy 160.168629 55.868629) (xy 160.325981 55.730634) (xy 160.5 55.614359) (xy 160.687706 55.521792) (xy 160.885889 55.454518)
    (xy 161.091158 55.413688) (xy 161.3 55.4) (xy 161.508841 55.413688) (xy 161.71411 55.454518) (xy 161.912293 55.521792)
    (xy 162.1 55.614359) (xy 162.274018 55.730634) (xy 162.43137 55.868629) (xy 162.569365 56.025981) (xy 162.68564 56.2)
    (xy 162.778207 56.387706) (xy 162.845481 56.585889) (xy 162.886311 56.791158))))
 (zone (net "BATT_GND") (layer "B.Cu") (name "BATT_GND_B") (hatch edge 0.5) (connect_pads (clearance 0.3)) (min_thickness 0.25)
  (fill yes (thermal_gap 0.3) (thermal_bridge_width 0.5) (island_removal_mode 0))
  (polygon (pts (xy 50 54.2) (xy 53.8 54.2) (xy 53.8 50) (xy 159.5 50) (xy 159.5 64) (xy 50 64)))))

